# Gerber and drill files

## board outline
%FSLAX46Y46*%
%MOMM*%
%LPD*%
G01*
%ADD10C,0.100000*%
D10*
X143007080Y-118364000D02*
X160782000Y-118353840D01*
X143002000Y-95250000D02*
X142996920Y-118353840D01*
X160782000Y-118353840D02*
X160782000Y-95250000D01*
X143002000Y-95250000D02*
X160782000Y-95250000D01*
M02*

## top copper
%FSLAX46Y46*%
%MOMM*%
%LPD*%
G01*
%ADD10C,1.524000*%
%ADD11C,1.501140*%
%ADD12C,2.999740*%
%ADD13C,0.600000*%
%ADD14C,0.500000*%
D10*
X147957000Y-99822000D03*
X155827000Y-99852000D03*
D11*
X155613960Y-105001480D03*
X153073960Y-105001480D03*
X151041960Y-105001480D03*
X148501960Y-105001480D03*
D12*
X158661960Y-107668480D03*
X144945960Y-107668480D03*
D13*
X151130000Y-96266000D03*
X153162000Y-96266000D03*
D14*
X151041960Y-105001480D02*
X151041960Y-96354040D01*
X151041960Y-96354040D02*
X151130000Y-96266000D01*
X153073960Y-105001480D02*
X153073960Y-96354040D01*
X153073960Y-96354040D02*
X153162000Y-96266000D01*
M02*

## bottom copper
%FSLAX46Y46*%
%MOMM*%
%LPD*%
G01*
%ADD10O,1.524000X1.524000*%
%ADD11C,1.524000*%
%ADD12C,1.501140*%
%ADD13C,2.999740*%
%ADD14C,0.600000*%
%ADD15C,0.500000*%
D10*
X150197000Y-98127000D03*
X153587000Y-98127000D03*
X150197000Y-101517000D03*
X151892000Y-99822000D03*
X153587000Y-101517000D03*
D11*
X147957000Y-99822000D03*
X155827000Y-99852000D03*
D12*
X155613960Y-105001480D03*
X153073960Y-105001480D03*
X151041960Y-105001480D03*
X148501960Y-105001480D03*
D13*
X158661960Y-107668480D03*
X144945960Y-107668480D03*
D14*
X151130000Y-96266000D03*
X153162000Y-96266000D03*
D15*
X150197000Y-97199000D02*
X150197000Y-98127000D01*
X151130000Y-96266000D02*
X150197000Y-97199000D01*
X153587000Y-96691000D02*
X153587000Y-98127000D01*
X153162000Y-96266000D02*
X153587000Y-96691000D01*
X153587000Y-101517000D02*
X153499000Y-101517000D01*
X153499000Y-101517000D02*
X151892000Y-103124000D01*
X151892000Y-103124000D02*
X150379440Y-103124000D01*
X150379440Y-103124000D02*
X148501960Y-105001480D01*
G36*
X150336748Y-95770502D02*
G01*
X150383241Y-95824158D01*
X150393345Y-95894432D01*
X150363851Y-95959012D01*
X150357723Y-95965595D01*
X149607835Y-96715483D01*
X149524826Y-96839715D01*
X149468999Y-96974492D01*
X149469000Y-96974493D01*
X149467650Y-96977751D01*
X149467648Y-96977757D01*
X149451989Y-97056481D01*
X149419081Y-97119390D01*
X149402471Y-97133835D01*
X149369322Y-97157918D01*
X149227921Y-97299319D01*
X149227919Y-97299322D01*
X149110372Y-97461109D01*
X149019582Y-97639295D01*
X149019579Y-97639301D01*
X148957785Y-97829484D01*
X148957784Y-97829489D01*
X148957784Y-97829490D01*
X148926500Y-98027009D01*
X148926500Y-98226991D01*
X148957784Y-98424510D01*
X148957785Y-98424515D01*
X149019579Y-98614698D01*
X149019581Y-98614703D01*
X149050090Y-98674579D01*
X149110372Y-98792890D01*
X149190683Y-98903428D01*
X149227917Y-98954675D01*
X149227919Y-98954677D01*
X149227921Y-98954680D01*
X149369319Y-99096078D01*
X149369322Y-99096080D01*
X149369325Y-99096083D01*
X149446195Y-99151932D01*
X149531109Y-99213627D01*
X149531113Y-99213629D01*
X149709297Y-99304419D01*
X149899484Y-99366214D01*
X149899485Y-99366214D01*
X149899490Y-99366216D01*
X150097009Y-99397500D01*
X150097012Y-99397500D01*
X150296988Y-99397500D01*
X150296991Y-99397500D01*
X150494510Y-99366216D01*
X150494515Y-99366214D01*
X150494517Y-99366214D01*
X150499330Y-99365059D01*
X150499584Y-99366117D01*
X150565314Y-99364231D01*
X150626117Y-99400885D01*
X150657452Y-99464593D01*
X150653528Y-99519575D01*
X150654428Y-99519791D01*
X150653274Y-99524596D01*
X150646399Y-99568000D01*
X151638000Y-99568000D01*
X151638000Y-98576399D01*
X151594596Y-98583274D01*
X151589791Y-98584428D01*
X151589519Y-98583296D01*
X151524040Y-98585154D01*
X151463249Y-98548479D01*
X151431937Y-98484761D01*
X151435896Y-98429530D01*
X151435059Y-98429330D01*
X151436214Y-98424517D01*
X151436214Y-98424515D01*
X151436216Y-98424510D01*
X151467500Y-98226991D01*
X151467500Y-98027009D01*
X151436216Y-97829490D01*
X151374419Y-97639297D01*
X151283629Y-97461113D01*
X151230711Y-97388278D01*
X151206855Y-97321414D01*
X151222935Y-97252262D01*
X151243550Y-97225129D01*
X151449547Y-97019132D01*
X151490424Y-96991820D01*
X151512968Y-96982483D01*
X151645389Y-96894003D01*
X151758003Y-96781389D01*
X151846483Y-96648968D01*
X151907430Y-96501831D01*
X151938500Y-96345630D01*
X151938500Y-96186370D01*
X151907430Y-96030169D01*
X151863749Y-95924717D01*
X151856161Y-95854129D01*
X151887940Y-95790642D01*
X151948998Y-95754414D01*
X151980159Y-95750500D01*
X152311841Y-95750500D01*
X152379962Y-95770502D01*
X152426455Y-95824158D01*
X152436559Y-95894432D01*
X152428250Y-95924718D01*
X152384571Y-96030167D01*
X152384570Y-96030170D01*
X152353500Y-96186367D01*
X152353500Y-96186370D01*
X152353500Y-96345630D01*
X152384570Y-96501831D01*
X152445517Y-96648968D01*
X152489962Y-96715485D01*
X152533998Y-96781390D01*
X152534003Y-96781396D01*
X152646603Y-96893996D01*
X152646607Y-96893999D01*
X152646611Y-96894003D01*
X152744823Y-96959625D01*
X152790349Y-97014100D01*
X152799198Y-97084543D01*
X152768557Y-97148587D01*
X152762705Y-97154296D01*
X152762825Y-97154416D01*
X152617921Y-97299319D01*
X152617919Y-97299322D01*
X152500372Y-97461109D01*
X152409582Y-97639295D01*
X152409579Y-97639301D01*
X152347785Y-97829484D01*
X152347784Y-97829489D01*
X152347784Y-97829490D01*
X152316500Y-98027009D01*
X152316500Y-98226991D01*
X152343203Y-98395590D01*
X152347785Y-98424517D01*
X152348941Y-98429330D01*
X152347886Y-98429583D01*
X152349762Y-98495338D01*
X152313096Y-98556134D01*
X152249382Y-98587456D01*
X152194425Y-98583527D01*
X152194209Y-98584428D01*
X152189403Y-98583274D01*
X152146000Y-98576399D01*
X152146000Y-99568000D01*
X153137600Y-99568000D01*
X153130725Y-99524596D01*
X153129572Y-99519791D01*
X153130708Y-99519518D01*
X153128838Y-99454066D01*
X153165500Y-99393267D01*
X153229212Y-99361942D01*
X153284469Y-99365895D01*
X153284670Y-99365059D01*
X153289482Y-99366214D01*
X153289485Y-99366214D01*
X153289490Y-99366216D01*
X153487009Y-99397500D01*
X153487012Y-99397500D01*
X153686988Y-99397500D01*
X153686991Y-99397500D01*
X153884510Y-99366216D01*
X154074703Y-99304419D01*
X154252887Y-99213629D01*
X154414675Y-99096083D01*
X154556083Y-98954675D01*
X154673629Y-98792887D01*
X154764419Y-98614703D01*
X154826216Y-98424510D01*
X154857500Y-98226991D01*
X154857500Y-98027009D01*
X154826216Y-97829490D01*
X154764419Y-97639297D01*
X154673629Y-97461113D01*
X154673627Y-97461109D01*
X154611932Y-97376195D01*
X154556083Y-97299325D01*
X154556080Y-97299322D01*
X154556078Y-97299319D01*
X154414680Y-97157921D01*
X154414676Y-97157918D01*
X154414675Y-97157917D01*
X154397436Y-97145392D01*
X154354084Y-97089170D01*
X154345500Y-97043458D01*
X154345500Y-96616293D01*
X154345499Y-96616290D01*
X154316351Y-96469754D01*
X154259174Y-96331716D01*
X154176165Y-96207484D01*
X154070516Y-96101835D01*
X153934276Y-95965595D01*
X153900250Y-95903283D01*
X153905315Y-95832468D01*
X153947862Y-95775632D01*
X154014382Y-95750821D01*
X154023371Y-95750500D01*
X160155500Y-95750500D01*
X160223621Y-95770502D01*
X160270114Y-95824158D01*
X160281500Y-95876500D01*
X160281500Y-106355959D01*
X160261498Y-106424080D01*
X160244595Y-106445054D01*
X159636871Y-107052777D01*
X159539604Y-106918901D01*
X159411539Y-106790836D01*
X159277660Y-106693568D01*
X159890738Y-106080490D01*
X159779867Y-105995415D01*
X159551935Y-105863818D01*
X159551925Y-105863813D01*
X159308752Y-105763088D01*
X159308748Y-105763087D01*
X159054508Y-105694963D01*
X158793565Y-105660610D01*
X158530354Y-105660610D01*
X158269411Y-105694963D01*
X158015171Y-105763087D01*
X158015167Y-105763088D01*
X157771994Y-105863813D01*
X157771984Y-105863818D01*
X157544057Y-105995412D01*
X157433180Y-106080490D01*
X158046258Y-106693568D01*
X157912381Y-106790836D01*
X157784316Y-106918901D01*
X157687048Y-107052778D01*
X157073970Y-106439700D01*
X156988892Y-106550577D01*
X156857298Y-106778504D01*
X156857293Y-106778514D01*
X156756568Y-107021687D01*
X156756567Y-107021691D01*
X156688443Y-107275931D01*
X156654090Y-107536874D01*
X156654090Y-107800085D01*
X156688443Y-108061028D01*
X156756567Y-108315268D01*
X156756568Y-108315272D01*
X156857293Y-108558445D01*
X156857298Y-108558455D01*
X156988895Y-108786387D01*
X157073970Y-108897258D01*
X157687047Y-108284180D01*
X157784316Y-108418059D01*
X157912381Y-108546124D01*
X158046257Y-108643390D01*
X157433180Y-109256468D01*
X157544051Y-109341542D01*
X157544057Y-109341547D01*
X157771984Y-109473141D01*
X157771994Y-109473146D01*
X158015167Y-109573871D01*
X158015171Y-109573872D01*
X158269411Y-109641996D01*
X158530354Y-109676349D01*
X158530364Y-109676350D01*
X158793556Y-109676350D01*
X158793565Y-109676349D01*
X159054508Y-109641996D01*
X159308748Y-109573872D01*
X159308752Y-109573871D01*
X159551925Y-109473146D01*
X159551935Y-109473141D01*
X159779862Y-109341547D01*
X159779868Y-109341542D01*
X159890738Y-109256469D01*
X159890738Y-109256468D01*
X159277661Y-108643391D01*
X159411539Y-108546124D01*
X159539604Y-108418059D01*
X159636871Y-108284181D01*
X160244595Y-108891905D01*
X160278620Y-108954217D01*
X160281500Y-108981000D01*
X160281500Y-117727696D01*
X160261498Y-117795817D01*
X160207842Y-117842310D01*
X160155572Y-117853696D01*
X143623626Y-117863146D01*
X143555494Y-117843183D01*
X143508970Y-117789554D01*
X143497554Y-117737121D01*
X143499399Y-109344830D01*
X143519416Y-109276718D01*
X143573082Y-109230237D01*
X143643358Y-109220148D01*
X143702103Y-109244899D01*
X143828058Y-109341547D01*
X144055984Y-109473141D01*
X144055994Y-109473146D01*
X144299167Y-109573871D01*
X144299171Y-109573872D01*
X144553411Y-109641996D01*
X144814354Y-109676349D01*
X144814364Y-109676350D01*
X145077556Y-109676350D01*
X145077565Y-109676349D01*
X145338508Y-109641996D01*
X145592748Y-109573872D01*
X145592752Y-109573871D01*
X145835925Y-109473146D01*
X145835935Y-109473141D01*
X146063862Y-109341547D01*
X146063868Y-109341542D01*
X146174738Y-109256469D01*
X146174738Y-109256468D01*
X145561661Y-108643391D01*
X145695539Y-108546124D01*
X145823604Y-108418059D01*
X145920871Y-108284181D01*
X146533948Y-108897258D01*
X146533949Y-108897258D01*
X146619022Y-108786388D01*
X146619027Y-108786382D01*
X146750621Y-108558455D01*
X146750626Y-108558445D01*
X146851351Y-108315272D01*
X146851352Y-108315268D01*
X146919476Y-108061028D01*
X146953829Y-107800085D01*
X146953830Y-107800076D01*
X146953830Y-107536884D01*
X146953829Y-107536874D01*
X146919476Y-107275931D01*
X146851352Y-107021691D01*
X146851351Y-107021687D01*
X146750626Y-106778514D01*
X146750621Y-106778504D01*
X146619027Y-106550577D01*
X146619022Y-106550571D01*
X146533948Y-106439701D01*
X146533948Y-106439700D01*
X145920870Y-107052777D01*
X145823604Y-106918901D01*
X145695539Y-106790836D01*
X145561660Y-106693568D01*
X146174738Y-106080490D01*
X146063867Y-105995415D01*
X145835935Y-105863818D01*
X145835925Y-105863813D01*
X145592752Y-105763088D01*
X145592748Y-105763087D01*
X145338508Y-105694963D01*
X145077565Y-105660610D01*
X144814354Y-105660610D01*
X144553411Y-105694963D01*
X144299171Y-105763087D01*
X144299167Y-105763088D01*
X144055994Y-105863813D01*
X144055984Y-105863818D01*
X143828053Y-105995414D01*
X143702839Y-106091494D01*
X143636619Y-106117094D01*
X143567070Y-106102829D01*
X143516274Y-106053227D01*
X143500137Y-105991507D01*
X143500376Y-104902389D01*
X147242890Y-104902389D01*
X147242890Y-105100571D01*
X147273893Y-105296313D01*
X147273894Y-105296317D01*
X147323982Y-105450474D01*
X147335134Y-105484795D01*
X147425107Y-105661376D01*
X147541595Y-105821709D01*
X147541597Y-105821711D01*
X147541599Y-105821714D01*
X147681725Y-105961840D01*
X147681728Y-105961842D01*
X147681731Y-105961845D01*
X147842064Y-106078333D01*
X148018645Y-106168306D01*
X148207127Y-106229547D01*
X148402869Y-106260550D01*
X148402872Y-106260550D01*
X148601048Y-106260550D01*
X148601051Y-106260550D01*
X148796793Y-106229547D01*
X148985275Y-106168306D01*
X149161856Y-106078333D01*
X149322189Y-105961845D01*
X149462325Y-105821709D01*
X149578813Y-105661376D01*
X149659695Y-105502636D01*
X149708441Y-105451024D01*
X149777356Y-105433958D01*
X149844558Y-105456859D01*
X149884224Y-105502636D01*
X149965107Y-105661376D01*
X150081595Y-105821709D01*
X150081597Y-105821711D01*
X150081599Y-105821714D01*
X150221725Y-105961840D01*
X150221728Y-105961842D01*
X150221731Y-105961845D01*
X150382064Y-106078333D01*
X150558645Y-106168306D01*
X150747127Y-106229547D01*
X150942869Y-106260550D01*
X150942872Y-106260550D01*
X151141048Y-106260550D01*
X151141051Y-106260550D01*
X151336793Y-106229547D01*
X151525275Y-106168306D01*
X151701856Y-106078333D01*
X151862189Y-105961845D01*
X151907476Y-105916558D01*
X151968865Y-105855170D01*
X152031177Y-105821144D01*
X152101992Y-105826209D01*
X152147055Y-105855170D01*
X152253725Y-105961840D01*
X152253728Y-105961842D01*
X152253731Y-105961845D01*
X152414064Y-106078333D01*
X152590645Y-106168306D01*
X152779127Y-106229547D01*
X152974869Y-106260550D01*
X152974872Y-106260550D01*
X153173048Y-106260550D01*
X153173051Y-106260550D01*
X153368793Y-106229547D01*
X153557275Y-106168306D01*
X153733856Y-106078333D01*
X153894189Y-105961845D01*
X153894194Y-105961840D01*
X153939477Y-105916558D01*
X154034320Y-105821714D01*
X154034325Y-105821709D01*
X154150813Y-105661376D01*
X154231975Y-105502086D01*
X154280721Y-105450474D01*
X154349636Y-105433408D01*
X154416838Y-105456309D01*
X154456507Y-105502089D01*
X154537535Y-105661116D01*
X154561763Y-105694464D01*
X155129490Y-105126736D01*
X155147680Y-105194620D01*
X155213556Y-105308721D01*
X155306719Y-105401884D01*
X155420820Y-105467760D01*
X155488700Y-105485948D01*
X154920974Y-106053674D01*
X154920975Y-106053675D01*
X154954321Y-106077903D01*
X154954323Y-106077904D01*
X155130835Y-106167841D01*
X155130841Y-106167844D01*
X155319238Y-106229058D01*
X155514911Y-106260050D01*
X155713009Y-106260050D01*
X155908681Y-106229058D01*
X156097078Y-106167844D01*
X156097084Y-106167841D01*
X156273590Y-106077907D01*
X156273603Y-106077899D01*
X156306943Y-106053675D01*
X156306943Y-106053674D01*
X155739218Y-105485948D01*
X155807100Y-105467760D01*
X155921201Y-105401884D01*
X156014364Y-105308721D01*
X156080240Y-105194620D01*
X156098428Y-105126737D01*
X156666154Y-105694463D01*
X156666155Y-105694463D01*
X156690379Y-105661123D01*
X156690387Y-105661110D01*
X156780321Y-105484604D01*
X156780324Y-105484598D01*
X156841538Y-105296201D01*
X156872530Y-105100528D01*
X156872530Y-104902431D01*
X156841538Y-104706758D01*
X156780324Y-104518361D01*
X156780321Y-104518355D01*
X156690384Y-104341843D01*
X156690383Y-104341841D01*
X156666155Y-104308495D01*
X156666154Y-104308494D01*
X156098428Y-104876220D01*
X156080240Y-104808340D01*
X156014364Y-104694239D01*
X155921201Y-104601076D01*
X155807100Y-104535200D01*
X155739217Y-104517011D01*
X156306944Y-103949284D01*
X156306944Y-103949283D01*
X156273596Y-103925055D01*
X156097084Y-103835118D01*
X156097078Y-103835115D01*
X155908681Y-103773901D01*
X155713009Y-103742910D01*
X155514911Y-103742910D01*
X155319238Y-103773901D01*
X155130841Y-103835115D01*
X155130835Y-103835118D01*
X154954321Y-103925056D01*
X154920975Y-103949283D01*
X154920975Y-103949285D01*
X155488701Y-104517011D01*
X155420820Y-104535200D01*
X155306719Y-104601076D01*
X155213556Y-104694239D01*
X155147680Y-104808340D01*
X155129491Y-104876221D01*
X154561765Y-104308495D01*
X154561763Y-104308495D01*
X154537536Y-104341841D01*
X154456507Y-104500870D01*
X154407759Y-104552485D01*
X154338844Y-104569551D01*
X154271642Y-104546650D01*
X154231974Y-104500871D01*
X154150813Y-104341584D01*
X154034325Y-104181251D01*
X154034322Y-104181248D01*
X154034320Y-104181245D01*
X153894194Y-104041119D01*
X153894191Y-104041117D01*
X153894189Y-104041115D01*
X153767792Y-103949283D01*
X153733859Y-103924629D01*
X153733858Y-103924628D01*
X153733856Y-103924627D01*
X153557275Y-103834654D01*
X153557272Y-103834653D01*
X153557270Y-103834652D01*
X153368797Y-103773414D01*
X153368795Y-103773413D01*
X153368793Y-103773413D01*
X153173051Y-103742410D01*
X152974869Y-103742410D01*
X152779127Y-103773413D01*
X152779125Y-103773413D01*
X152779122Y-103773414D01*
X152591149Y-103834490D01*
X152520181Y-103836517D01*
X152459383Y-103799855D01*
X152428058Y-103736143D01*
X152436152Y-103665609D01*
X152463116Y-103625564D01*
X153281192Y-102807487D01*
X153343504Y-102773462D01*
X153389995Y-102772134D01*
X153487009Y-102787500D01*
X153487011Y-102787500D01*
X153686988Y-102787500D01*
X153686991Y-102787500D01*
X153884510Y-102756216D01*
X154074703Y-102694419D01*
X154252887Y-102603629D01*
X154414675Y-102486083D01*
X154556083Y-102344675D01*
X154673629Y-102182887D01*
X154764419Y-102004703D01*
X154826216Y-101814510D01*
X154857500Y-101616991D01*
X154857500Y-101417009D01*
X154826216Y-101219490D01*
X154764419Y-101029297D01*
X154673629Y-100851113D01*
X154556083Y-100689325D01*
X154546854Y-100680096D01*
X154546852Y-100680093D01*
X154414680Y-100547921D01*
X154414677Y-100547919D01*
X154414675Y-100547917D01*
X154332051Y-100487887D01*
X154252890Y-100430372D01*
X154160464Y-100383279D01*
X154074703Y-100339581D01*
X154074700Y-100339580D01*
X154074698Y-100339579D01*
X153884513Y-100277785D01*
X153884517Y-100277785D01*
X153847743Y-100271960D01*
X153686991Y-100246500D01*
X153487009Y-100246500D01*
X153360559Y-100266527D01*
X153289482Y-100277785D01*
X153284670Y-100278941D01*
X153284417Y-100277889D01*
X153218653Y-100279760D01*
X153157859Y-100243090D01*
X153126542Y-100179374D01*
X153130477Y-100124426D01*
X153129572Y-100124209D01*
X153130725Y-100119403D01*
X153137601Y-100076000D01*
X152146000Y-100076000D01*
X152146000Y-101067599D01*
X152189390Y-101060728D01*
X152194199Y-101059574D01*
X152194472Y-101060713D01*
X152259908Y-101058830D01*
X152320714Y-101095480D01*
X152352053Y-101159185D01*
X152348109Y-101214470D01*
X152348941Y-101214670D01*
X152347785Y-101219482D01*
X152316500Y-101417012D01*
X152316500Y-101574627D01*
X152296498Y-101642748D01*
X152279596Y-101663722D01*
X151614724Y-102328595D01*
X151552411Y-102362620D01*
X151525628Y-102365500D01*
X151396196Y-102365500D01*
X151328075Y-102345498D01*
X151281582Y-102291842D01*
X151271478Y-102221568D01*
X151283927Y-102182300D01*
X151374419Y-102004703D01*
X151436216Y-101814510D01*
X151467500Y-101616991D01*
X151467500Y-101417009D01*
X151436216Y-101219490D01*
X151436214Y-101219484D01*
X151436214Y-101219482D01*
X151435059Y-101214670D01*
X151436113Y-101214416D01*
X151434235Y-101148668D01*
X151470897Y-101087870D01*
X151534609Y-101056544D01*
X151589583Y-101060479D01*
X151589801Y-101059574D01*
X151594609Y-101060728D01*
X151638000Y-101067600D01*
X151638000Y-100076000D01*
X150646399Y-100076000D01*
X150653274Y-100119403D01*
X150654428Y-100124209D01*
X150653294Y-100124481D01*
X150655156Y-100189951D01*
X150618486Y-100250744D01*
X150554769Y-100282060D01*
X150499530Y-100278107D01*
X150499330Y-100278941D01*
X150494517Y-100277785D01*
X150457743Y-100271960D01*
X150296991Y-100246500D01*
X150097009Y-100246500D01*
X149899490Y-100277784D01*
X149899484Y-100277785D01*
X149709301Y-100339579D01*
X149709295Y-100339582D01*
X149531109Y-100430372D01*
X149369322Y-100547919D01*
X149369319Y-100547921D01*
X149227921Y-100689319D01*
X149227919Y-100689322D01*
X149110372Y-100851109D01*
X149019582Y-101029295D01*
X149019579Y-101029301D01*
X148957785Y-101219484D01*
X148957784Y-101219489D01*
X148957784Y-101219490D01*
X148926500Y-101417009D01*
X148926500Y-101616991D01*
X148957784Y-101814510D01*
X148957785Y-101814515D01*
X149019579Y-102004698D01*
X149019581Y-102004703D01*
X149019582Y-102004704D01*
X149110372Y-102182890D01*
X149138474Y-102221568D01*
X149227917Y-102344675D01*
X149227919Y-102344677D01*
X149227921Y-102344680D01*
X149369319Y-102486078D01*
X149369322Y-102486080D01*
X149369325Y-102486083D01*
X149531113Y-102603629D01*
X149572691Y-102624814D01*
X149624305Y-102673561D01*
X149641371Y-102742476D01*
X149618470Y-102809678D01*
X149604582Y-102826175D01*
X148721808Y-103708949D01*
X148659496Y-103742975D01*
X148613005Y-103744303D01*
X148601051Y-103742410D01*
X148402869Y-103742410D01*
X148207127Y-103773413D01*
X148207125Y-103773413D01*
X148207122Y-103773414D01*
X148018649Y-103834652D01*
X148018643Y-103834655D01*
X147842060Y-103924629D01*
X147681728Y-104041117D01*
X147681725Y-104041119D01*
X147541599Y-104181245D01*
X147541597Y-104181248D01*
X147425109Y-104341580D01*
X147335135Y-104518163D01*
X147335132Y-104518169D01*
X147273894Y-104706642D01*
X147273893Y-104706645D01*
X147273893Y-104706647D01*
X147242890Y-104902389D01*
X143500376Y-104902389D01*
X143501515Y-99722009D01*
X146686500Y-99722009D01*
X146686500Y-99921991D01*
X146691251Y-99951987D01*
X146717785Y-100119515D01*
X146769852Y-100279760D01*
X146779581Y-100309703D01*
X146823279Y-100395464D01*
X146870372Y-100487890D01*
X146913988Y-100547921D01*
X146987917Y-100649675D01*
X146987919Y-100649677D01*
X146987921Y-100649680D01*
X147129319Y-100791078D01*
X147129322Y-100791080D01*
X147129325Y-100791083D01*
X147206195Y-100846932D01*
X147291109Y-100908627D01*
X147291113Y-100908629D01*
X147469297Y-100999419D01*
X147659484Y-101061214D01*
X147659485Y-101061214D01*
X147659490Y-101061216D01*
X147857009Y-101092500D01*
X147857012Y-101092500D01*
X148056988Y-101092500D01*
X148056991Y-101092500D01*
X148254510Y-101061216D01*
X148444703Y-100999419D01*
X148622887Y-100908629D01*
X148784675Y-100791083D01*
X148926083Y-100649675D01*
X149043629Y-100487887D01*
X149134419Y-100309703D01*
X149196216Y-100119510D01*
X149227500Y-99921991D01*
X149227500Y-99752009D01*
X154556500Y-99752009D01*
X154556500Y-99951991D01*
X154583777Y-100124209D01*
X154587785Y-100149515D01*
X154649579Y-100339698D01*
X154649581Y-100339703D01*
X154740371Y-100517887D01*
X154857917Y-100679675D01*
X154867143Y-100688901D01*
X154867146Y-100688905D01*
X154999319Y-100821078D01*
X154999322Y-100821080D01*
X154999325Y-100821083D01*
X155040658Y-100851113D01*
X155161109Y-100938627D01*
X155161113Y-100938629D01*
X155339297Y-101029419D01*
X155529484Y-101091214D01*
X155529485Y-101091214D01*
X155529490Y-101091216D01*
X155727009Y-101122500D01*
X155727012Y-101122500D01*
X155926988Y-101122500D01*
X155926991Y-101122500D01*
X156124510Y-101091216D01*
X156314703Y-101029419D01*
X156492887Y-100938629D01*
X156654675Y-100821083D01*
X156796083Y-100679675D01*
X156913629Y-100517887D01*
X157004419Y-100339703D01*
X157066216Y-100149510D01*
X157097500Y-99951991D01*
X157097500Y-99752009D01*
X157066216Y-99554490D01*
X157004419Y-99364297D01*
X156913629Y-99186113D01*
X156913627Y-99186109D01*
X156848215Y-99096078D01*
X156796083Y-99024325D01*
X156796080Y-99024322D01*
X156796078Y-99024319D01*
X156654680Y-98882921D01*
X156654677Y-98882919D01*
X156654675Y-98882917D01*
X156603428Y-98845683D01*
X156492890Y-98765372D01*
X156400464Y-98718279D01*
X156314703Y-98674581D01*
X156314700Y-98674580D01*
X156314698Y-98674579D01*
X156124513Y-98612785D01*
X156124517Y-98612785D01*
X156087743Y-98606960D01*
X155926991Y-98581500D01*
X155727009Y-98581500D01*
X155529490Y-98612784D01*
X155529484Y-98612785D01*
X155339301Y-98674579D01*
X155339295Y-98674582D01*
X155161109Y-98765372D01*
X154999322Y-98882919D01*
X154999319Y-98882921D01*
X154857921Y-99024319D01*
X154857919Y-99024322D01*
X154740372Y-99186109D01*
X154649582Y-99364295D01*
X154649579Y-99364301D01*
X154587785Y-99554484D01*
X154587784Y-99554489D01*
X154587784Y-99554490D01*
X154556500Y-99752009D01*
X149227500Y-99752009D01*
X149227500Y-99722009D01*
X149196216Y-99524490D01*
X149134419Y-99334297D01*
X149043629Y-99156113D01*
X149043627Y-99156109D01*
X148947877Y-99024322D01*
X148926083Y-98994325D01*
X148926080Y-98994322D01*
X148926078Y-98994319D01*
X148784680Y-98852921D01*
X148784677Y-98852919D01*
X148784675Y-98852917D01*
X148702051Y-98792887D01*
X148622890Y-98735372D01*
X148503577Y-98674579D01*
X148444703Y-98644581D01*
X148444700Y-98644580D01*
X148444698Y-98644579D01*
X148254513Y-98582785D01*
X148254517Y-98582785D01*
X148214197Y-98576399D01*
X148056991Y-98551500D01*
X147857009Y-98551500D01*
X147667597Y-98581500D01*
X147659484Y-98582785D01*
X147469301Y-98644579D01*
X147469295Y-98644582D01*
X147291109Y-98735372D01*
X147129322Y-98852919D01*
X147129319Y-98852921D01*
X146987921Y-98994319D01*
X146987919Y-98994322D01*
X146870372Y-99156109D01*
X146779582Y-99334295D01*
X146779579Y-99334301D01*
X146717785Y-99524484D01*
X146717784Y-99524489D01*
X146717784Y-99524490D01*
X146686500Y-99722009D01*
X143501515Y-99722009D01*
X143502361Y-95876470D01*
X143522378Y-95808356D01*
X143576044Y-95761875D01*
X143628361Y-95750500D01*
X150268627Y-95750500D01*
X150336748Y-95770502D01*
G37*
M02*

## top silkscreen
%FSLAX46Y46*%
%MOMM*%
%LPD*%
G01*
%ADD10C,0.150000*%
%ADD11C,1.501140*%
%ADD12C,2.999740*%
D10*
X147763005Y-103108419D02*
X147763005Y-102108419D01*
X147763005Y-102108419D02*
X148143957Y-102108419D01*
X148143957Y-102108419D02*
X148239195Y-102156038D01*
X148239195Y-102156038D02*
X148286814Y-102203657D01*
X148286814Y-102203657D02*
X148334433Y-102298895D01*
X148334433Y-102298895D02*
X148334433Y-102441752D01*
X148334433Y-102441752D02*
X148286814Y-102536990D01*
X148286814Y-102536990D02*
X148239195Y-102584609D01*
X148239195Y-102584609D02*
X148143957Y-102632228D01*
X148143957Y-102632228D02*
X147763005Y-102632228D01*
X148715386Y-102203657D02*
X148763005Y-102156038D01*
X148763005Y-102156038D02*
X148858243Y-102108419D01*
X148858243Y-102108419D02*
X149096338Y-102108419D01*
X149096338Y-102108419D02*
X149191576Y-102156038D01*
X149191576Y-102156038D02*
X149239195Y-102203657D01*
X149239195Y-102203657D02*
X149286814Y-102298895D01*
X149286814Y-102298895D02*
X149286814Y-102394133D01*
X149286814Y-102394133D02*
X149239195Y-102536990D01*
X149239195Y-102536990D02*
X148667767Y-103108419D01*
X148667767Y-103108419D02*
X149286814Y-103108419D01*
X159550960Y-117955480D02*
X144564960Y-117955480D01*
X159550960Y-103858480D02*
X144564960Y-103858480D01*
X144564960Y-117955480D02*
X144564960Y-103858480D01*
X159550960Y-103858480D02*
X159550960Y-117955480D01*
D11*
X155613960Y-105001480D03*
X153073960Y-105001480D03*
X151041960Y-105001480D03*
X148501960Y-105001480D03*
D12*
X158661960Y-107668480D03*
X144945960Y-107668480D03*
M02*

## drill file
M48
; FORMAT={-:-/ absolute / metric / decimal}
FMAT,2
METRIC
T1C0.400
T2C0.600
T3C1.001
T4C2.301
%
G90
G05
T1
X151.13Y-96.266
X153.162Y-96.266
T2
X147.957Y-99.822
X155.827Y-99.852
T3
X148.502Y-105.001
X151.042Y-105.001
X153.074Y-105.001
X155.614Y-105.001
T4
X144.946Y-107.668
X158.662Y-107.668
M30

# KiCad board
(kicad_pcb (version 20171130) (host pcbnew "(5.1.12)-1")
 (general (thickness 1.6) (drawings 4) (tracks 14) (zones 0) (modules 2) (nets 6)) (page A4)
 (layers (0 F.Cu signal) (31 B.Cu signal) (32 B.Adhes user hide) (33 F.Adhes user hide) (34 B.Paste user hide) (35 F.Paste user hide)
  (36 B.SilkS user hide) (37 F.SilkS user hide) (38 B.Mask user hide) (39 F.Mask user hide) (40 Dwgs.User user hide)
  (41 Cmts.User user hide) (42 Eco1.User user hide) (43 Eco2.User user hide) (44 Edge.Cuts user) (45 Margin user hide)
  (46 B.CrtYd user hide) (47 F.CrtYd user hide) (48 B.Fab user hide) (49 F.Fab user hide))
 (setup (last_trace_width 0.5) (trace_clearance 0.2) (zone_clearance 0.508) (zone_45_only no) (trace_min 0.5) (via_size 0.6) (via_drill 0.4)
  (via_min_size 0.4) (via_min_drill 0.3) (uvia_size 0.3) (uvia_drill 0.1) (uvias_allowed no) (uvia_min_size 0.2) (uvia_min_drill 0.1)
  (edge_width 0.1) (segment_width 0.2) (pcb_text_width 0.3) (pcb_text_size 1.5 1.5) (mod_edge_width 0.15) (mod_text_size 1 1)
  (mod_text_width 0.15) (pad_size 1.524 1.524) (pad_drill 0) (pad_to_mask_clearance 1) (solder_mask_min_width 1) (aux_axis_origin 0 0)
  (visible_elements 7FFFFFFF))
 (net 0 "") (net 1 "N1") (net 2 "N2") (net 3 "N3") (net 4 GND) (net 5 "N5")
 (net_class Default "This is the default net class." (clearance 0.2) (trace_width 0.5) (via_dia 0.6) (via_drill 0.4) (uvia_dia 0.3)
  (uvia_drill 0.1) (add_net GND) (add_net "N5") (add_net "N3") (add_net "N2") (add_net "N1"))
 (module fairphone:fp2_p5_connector (layer B.Cu) (at 151.892 99.822)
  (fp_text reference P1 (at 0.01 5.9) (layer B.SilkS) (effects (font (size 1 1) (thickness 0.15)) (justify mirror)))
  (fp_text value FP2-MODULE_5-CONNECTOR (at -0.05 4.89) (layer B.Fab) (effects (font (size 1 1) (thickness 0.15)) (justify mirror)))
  (pad 5 smd oval (at -1.695 -1.695) (size 1.524 1.524) (layers B.Cu B.Paste B.Mask) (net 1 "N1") (solder_mask_margin 1))
  (pad 4 smd oval (at 1.695 -1.695) (size 1.524 1.524) (layers B.Cu B.Paste) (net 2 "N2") (solder_mask_margin 1))
  (pad 2 smd oval (at -1.695 1.695) (size 1.524 1.524) (layers B.Cu B.Paste B.Mask) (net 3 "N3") (solder_mask_margin 1))
  (pad 3 smd oval (at 0 0) (size 1.524 1.524) (layers B.Cu B.Paste B.Mask) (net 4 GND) (solder_mask_margin 1))
  (pad 1 smd oval (at 1.695 1.695) (size 1.524 1.524) (layers B.Cu B.Paste B.Mask) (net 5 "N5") (solder_mask_margin 1))
  (pad "" thru_hole circle (at -3.935 0) (size 1.524 1.524) (drill 0.6) (layers *.Cu *.Mask B.SilkS))
  (pad "" thru_hole circle (at 3.935 0.03) (size 1.524 1.524) (drill 0.6) (layers *.Cu *.Mask B.SilkS)))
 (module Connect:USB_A (layer F.Cu) (at 148.5011 105.0036)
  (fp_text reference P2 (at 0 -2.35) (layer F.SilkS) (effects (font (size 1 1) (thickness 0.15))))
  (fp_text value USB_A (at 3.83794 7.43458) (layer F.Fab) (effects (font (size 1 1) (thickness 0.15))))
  (fp_line (start 11.04986 12.95188) (end -3.93614 12.95188) (layer F.SilkS) (width 0.15))
  (fp_line (start 11.04986 -1.14512) (end -3.93614 -1.14512) (layer F.SilkS) (width 0.15))
  (fp_line (start -3.93614 12.95188) (end -3.93614 -1.14512) (layer F.SilkS) (width 0.15))
  (fp_line (start 11.04986 -1.14512) (end 11.04986 12.95188) (layer F.SilkS) (width 0.15))
  (pad 4 thru_hole circle (at 7.11286 -0.00212 270) (size 1.50114 1.50114) (drill 1.00076) (layers *.Cu *.Mask F.SilkS) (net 4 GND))
  (pad 3 thru_hole circle (at 4.57286 -0.00212 270) (size 1.50114 1.50114) (drill 1.00076) (layers *.Cu *.Mask F.SilkS) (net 2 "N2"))
  (pad 2 thru_hole circle (at 2.54086 -0.00212 270) (size 1.50114 1.50114) (drill 1.00076) (layers *.Cu *.Mask F.SilkS) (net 1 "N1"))
  (pad 1 thru_hole circle (at 0.00086 -0.00212 270) (size 1.50114 1.50114) (drill 1.00076) (layers *.Cu *.Mask F.SilkS) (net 5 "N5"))
  (pad 5 thru_hole circle (at 10.16086 2.66488 270) (size 2.99974 2.99974) (drill 2.30124) (layers *.Cu *.Mask F.SilkS) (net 4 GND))
  (pad 5 thru_hole circle (at -3.55514 2.66488 270) (size 2.99974 2.99974) (drill 2.30124) (layers *.Cu *.Mask F.SilkS) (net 4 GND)))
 (gr_line (start 143.00708 118.364) (end 160.782 118.35384) (layer Edge.Cuts) (width 0.1))
 (gr_line (start 143.002 95.25) (end 142.99692 118.35384) (angle 90) (layer Edge.Cuts) (width 0.1))
 (gr_line (start 160.782 118.35384) (end 160.782 95.25) (angle 90) (layer Edge.Cuts) (width 0.1))
 (gr_line (start 143.002 95.25) (end 160.782 95.25) (angle 90) (layer Edge.Cuts) (width 0.1))
 (segment (start 151.04196 105.00148) (end 151.04196 96.35404) (width 0.5) (layer F.Cu) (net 1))
 (segment (start 151.04196 96.35404) (end 151.13 96.266) (width 0.5) (layer F.Cu) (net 1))
 (segment (start 150.197 97.199) (end 150.197 98.127) (width 0.5) (layer B.Cu) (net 1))
 (segment (start 151.13 96.266) (end 150.197 97.199) (width 0.5) (layer B.Cu) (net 1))
 (via (at 151.13 96.266) (size 0.6) (drill 0.4) (layers F.Cu B.Cu) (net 1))
 (segment (start 153.07396 105.00148) (end 153.07396 96.35404) (width 0.5) (layer F.Cu) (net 2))
 (segment (start 153.587 96.691) (end 153.587 98.127) (width 0.5) (layer B.Cu) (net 2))
 (segment (start 153.162 96.266) (end 153.587 96.691) (width 0.5) (layer B.Cu) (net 2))
 (via (at 153.162 96.266) (size 0.6) (drill 0.4) (layers F.Cu B.Cu) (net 2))
 (segment (start 153.07396 96.35404) (end 153.162 96.266) (width 0.5) (layer F.Cu) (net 2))
 (segment (start 153.587 101.517) (end 153.499 101.517) (width 0.5) (layer B.Cu) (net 5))
 (segment (start 153.499 101.517) (end 151.892 103.124) (width 0.5) (layer B.Cu) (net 5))
 (segment (start 151.892 103.124) (end 150.37944 103.124) (width 0.5) (layer B.Cu) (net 5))
 (segment (start 150.37944 103.124) (end 148.50196 105.00148) (width 0.5) (layer B.Cu) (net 5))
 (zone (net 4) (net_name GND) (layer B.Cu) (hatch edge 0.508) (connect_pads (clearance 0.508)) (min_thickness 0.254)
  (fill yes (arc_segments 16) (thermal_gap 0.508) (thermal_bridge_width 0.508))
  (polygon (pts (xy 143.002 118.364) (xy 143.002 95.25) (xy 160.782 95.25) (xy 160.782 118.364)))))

